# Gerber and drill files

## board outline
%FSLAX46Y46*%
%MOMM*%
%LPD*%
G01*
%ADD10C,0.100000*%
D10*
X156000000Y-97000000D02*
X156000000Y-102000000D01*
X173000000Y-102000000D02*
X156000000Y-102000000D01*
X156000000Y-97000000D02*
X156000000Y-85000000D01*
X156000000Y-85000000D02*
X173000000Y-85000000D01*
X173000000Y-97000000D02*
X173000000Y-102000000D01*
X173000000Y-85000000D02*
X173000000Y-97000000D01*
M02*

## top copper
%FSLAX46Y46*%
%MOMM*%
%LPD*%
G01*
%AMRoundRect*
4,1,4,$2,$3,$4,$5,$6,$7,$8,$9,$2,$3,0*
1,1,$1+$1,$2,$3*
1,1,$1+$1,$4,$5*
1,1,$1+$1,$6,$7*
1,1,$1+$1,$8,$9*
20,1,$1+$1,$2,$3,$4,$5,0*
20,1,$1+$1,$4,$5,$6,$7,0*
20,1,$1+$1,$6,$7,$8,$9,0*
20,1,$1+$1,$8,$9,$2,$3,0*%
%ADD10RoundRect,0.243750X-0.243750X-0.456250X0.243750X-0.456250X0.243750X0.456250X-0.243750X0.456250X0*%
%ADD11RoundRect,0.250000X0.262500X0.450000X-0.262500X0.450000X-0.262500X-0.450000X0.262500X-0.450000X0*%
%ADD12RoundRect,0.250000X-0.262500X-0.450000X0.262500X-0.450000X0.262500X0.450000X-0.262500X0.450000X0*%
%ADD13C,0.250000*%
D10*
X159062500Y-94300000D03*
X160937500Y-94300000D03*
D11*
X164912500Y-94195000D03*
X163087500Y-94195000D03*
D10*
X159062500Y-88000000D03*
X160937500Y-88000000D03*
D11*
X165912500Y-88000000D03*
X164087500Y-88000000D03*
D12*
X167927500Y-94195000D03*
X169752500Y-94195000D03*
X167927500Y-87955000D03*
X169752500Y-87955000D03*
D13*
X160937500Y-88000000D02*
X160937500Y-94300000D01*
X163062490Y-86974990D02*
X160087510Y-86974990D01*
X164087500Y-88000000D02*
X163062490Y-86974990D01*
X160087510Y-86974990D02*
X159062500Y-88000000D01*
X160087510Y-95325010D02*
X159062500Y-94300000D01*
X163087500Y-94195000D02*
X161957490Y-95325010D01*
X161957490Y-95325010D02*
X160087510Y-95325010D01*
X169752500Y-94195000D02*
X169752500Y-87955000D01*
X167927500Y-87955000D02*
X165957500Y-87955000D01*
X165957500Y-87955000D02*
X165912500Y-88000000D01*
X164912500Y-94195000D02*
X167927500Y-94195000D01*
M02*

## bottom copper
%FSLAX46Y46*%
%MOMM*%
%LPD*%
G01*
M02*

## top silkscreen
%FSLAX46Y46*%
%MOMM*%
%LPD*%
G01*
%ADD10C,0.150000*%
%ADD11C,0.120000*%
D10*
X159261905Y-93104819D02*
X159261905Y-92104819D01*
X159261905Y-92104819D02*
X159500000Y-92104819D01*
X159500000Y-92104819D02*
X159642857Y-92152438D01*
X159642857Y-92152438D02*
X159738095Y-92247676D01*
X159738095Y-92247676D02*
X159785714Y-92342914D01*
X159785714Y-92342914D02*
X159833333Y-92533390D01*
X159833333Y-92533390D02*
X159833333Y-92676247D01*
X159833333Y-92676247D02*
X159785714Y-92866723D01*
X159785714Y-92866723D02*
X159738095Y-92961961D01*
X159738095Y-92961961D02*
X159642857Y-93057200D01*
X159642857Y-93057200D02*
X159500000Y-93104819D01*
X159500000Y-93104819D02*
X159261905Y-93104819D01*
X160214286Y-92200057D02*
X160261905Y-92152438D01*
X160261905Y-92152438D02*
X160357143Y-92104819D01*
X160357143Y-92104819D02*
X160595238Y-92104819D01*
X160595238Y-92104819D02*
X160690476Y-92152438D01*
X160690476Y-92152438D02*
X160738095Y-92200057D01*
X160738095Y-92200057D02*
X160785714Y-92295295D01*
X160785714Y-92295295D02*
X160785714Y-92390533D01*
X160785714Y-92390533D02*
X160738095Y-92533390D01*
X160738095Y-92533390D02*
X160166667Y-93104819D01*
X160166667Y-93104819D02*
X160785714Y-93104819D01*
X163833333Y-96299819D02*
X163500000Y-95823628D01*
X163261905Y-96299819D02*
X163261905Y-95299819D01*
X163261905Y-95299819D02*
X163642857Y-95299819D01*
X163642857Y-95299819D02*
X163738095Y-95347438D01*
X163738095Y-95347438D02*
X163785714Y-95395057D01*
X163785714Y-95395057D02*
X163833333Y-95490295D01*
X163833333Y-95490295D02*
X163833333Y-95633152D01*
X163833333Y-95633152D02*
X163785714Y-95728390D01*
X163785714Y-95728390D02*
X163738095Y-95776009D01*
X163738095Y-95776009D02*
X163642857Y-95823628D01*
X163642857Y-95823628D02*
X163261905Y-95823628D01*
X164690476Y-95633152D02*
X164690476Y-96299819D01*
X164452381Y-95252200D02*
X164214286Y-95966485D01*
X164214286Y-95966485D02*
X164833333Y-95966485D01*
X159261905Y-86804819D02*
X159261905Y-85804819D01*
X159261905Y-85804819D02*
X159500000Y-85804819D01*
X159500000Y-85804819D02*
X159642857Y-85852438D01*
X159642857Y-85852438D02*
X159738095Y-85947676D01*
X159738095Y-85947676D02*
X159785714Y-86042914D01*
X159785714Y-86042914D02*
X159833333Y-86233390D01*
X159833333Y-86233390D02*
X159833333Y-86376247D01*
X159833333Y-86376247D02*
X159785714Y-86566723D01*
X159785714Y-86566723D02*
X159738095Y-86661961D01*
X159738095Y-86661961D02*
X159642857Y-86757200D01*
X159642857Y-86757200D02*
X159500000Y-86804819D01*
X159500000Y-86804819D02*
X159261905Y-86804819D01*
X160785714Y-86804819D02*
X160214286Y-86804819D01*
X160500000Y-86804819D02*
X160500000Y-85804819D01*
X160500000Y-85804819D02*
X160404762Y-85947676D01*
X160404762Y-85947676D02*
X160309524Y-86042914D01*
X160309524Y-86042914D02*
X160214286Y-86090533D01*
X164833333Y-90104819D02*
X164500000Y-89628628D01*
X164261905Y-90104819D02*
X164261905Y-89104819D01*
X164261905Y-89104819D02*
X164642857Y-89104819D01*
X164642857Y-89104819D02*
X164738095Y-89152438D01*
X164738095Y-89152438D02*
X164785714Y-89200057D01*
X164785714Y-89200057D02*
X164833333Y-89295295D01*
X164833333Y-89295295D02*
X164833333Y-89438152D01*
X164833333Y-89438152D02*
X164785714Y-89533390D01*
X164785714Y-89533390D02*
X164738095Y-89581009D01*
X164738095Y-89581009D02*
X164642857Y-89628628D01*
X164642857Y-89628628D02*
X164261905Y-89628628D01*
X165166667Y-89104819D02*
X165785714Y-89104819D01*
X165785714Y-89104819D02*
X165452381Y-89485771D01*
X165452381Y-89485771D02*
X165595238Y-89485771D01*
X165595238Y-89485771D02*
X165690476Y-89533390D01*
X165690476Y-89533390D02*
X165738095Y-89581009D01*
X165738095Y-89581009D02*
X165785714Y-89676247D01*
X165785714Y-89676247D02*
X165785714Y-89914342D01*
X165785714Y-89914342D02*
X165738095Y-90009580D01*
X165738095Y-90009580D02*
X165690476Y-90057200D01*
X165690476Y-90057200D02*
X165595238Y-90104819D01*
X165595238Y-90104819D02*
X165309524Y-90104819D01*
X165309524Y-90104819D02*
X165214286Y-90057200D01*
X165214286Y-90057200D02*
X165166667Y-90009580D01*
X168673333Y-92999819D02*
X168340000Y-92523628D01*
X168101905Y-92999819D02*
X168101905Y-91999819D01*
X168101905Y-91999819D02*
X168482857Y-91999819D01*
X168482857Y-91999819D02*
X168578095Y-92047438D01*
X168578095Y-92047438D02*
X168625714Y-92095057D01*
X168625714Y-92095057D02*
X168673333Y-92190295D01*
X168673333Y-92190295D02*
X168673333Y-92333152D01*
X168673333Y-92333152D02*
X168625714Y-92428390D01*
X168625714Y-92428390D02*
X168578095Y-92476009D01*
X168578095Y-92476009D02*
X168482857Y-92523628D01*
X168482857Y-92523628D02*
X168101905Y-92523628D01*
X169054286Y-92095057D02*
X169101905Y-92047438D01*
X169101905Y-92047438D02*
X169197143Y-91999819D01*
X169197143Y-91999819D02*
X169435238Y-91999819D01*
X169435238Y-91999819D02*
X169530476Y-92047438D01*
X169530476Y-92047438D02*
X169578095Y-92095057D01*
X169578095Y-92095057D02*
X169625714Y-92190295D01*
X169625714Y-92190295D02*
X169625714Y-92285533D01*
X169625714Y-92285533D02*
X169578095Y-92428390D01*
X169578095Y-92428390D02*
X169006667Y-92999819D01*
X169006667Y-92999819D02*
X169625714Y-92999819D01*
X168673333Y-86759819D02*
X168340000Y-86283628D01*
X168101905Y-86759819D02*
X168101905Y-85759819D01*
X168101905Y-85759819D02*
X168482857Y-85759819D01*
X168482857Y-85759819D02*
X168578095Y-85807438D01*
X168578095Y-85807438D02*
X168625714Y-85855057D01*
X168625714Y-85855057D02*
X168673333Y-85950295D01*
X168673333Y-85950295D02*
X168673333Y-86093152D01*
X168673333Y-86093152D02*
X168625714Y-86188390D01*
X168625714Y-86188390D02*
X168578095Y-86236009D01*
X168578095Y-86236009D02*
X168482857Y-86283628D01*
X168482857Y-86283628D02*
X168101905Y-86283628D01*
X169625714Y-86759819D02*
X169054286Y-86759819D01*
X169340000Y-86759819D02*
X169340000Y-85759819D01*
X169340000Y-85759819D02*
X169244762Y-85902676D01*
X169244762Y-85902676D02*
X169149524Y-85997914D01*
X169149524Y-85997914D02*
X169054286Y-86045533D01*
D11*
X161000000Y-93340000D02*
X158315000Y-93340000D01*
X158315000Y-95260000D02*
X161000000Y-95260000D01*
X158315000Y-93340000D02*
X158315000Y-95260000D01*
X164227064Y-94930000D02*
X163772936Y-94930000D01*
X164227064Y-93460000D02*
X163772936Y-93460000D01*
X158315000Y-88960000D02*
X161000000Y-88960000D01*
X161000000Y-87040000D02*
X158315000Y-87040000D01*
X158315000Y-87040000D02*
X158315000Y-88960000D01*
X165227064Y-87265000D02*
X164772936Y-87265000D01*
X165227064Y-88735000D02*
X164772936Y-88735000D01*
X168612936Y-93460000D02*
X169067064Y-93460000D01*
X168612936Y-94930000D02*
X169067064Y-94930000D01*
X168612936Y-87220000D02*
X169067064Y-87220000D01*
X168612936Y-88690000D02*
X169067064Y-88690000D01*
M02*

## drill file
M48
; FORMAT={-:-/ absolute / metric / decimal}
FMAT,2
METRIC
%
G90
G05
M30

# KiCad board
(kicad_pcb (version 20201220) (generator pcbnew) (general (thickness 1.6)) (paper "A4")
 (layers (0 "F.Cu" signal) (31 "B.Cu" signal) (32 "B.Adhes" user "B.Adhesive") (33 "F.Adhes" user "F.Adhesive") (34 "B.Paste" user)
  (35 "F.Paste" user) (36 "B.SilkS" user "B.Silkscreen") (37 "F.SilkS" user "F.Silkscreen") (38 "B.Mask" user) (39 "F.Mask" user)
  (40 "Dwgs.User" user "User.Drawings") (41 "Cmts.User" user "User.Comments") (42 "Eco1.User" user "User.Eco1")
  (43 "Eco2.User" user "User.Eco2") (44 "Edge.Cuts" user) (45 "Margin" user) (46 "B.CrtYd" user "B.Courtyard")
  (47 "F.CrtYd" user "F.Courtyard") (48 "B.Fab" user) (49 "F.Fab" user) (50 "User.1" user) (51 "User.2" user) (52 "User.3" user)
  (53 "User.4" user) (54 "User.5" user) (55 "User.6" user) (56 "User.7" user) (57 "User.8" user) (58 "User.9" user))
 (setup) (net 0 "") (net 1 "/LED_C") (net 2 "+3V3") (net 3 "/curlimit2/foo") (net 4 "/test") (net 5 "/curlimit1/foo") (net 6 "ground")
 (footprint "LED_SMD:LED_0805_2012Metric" (layer "F.Cu") (at 160 94.3)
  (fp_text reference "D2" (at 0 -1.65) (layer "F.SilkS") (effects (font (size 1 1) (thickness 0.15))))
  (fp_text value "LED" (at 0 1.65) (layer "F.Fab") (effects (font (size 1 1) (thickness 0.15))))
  (fp_line (start 1 -0.96) (end -1.685 -0.96) (layer "F.SilkS") (width 0.12))
  (fp_line (start -1.685 0.96) (end 1 0.96) (layer "F.SilkS") (width 0.12))
  (fp_line (start -1.685 -0.96) (end -1.685 0.96) (layer "F.SilkS") (width 0.12))
  (pad "1" smd roundrect (at -0.9375 0) (size 0.975 1.4) (layers "F.Cu" "F.Paste" "F.Mask") (roundrect_rratio 0.25) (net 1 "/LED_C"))
  (pad "2" smd roundrect (at 0.9375 0) (size 0.975 1.4) (layers "F.Cu" "F.Paste" "F.Mask") (roundrect_rratio 0.25) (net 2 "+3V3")))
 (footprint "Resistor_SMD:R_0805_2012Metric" (layer "F.Cu") (at 164 94.195 180)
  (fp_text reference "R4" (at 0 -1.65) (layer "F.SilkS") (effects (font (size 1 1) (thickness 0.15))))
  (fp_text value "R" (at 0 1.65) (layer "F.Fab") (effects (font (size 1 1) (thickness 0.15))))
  (fp_line (start -0.227064 -0.735) (end 0.227064 -0.735) (layer "F.SilkS") (width 0.12))
  (fp_line (start -0.227064 0.735) (end 0.227064 0.735) (layer "F.SilkS") (width 0.12))
  (pad "1" smd roundrect (at -0.9125 0 180) (size 1.025 1.4) (layers "F.Cu" "F.Paste" "F.Mask") (roundrect_rratio 0.243902)
   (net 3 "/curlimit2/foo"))
  (pad "2" smd roundrect (at 0.9125 0 180) (size 1.025 1.4) (layers "F.Cu" "F.Paste" "F.Mask") (roundrect_rratio 0.243902) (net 1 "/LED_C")))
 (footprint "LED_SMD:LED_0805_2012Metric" (layer "F.Cu") (at 160 88)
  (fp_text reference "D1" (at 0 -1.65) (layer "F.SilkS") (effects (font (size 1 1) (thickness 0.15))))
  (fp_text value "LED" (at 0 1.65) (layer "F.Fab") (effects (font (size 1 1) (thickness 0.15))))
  (fp_line (start -1.685 0.96) (end 1 0.96) (layer "F.SilkS") (width 0.12))
  (fp_line (start 1 -0.96) (end -1.685 -0.96) (layer "F.SilkS") (width 0.12))
  (fp_line (start -1.685 -0.96) (end -1.685 0.96) (layer "F.SilkS") (width 0.12))
  (pad "1" smd roundrect (at -0.9375 0) (size 0.975 1.4) (layers "F.Cu" "F.Paste" "F.Mask") (roundrect_rratio 0.25) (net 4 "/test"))
  (pad "2" smd roundrect (at 0.9375 0) (size 0.975 1.4) (layers "F.Cu" "F.Paste" "F.Mask") (roundrect_rratio 0.25) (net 2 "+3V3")))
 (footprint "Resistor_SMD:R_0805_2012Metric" (layer "F.Cu") (at 165 88 180)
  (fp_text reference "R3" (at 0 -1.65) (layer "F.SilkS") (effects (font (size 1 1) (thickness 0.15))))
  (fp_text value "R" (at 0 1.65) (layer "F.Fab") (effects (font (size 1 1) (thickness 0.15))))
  (fp_line (start -0.227064 0.735) (end 0.227064 0.735) (layer "F.SilkS") (width 0.12))
  (fp_line (start -0.227064 -0.735) (end 0.227064 -0.735) (layer "F.SilkS") (width 0.12))
  (pad "1" smd roundrect (at -0.9125 0 180) (size 1.025 1.4) (layers "F.Cu" "F.Paste" "F.Mask") (roundrect_rratio 0.243902)
   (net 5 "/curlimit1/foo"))
  (pad "2" smd roundrect (at 0.9125 0 180) (size 1.025 1.4) (layers "F.Cu" "F.Paste" "F.Mask") (roundrect_rratio 0.243902) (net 4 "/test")))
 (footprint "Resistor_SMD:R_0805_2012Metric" (layer "F.Cu") (at 168.84 94.195)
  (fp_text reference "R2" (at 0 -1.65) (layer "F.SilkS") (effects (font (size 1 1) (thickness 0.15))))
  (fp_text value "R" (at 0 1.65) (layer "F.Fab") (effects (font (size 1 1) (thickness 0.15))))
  (fp_line (start -0.227064 -0.735) (end 0.227064 -0.735) (layer "F.SilkS") (width 0.12))
  (fp_line (start -0.227064 0.735) (end 0.227064 0.735) (layer "F.SilkS") (width 0.12))
  (pad "1" smd roundrect (at -0.9125 0) (size 1.025 1.4) (layers "F.Cu" "F.Paste" "F.Mask") (roundrect_rratio 0.243902)
   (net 3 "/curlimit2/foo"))
  (pad "2" smd roundrect (at 0.9125 0) (size 1.025 1.4) (layers "F.Cu" "F.Paste" "F.Mask") (roundrect_rratio 0.243902) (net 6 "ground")))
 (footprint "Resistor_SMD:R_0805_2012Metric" (layer "F.Cu") (at 168.84 87.955)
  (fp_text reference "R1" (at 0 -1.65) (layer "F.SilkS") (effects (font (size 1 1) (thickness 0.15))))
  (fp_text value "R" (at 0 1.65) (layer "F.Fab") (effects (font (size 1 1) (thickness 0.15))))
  (fp_line (start -0.227064 -0.735) (end 0.227064 -0.735) (layer "F.SilkS") (width 0.12))
  (fp_line (start -0.227064 0.735) (end 0.227064 0.735) (layer "F.SilkS") (width 0.12))
  (pad "1" smd roundrect (at -0.9125 0) (size 1.025 1.4) (layers "F.Cu" "F.Paste" "F.Mask") (roundrect_rratio 0.243902)
   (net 5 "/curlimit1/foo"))
  (pad "2" smd roundrect (at 0.9125 0) (size 1.025 1.4) (layers "F.Cu" "F.Paste" "F.Mask") (roundrect_rratio 0.243902) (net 6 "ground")))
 (gr_line (start 156 97) (end 156 102) (layer "Edge.Cuts") (width 0.1))
 (gr_line (start 173 102) (end 156 102) (layer "Edge.Cuts") (width 0.1))
 (gr_line (start 156 97) (end 156 85) (layer "Edge.Cuts") (width 0.1))
 (gr_line (start 156 85) (end 173 85) (layer "Edge.Cuts") (width 0.1))
 (gr_line (start 173 97) (end 173 102) (layer "Edge.Cuts") (width 0.1))
 (gr_line (start 173 85) (end 173 97) (layer "Edge.Cuts") (width 0.1))
 (segment (start 160.9375 88) (end 160.9375 94.3) (width 0.25) (layer "F.Cu") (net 2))
 (segment (start 163.06249 86.97499) (end 160.08751 86.97499) (width 0.25) (layer "F.Cu") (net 4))
 (segment (start 164.0875 88) (end 163.06249 86.97499) (width 0.25) (layer "F.Cu") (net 4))
 (segment (start 160.08751 86.97499) (end 159.0625 88) (width 0.25) (layer "F.Cu") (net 4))
 (segment (start 160.08751 95.32501) (end 159.0625 94.3) (width 0.25) (layer "F.Cu") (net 1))
 (segment (start 163.0875 94.195) (end 161.95749 95.32501) (width 0.25) (layer "F.Cu") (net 1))
 (segment (start 161.95749 95.32501) (end 160.08751 95.32501) (width 0.25) (layer "F.Cu") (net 1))
 (segment (start 169.7525 94.195) (end 169.7525 87.955) (width 0.25) (layer "F.Cu") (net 6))
 (segment (start 167.9275 87.955) (end 165.9575 87.955) (width 0.25) (layer "F.Cu") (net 5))
 (segment (start 165.9575 87.955) (end 165.9125 88) (width 0.25) (layer "F.Cu") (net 5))
 (segment (start 164.9125 94.195) (end 167.9275 94.195) (width 0.25) (layer "F.Cu") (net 3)))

